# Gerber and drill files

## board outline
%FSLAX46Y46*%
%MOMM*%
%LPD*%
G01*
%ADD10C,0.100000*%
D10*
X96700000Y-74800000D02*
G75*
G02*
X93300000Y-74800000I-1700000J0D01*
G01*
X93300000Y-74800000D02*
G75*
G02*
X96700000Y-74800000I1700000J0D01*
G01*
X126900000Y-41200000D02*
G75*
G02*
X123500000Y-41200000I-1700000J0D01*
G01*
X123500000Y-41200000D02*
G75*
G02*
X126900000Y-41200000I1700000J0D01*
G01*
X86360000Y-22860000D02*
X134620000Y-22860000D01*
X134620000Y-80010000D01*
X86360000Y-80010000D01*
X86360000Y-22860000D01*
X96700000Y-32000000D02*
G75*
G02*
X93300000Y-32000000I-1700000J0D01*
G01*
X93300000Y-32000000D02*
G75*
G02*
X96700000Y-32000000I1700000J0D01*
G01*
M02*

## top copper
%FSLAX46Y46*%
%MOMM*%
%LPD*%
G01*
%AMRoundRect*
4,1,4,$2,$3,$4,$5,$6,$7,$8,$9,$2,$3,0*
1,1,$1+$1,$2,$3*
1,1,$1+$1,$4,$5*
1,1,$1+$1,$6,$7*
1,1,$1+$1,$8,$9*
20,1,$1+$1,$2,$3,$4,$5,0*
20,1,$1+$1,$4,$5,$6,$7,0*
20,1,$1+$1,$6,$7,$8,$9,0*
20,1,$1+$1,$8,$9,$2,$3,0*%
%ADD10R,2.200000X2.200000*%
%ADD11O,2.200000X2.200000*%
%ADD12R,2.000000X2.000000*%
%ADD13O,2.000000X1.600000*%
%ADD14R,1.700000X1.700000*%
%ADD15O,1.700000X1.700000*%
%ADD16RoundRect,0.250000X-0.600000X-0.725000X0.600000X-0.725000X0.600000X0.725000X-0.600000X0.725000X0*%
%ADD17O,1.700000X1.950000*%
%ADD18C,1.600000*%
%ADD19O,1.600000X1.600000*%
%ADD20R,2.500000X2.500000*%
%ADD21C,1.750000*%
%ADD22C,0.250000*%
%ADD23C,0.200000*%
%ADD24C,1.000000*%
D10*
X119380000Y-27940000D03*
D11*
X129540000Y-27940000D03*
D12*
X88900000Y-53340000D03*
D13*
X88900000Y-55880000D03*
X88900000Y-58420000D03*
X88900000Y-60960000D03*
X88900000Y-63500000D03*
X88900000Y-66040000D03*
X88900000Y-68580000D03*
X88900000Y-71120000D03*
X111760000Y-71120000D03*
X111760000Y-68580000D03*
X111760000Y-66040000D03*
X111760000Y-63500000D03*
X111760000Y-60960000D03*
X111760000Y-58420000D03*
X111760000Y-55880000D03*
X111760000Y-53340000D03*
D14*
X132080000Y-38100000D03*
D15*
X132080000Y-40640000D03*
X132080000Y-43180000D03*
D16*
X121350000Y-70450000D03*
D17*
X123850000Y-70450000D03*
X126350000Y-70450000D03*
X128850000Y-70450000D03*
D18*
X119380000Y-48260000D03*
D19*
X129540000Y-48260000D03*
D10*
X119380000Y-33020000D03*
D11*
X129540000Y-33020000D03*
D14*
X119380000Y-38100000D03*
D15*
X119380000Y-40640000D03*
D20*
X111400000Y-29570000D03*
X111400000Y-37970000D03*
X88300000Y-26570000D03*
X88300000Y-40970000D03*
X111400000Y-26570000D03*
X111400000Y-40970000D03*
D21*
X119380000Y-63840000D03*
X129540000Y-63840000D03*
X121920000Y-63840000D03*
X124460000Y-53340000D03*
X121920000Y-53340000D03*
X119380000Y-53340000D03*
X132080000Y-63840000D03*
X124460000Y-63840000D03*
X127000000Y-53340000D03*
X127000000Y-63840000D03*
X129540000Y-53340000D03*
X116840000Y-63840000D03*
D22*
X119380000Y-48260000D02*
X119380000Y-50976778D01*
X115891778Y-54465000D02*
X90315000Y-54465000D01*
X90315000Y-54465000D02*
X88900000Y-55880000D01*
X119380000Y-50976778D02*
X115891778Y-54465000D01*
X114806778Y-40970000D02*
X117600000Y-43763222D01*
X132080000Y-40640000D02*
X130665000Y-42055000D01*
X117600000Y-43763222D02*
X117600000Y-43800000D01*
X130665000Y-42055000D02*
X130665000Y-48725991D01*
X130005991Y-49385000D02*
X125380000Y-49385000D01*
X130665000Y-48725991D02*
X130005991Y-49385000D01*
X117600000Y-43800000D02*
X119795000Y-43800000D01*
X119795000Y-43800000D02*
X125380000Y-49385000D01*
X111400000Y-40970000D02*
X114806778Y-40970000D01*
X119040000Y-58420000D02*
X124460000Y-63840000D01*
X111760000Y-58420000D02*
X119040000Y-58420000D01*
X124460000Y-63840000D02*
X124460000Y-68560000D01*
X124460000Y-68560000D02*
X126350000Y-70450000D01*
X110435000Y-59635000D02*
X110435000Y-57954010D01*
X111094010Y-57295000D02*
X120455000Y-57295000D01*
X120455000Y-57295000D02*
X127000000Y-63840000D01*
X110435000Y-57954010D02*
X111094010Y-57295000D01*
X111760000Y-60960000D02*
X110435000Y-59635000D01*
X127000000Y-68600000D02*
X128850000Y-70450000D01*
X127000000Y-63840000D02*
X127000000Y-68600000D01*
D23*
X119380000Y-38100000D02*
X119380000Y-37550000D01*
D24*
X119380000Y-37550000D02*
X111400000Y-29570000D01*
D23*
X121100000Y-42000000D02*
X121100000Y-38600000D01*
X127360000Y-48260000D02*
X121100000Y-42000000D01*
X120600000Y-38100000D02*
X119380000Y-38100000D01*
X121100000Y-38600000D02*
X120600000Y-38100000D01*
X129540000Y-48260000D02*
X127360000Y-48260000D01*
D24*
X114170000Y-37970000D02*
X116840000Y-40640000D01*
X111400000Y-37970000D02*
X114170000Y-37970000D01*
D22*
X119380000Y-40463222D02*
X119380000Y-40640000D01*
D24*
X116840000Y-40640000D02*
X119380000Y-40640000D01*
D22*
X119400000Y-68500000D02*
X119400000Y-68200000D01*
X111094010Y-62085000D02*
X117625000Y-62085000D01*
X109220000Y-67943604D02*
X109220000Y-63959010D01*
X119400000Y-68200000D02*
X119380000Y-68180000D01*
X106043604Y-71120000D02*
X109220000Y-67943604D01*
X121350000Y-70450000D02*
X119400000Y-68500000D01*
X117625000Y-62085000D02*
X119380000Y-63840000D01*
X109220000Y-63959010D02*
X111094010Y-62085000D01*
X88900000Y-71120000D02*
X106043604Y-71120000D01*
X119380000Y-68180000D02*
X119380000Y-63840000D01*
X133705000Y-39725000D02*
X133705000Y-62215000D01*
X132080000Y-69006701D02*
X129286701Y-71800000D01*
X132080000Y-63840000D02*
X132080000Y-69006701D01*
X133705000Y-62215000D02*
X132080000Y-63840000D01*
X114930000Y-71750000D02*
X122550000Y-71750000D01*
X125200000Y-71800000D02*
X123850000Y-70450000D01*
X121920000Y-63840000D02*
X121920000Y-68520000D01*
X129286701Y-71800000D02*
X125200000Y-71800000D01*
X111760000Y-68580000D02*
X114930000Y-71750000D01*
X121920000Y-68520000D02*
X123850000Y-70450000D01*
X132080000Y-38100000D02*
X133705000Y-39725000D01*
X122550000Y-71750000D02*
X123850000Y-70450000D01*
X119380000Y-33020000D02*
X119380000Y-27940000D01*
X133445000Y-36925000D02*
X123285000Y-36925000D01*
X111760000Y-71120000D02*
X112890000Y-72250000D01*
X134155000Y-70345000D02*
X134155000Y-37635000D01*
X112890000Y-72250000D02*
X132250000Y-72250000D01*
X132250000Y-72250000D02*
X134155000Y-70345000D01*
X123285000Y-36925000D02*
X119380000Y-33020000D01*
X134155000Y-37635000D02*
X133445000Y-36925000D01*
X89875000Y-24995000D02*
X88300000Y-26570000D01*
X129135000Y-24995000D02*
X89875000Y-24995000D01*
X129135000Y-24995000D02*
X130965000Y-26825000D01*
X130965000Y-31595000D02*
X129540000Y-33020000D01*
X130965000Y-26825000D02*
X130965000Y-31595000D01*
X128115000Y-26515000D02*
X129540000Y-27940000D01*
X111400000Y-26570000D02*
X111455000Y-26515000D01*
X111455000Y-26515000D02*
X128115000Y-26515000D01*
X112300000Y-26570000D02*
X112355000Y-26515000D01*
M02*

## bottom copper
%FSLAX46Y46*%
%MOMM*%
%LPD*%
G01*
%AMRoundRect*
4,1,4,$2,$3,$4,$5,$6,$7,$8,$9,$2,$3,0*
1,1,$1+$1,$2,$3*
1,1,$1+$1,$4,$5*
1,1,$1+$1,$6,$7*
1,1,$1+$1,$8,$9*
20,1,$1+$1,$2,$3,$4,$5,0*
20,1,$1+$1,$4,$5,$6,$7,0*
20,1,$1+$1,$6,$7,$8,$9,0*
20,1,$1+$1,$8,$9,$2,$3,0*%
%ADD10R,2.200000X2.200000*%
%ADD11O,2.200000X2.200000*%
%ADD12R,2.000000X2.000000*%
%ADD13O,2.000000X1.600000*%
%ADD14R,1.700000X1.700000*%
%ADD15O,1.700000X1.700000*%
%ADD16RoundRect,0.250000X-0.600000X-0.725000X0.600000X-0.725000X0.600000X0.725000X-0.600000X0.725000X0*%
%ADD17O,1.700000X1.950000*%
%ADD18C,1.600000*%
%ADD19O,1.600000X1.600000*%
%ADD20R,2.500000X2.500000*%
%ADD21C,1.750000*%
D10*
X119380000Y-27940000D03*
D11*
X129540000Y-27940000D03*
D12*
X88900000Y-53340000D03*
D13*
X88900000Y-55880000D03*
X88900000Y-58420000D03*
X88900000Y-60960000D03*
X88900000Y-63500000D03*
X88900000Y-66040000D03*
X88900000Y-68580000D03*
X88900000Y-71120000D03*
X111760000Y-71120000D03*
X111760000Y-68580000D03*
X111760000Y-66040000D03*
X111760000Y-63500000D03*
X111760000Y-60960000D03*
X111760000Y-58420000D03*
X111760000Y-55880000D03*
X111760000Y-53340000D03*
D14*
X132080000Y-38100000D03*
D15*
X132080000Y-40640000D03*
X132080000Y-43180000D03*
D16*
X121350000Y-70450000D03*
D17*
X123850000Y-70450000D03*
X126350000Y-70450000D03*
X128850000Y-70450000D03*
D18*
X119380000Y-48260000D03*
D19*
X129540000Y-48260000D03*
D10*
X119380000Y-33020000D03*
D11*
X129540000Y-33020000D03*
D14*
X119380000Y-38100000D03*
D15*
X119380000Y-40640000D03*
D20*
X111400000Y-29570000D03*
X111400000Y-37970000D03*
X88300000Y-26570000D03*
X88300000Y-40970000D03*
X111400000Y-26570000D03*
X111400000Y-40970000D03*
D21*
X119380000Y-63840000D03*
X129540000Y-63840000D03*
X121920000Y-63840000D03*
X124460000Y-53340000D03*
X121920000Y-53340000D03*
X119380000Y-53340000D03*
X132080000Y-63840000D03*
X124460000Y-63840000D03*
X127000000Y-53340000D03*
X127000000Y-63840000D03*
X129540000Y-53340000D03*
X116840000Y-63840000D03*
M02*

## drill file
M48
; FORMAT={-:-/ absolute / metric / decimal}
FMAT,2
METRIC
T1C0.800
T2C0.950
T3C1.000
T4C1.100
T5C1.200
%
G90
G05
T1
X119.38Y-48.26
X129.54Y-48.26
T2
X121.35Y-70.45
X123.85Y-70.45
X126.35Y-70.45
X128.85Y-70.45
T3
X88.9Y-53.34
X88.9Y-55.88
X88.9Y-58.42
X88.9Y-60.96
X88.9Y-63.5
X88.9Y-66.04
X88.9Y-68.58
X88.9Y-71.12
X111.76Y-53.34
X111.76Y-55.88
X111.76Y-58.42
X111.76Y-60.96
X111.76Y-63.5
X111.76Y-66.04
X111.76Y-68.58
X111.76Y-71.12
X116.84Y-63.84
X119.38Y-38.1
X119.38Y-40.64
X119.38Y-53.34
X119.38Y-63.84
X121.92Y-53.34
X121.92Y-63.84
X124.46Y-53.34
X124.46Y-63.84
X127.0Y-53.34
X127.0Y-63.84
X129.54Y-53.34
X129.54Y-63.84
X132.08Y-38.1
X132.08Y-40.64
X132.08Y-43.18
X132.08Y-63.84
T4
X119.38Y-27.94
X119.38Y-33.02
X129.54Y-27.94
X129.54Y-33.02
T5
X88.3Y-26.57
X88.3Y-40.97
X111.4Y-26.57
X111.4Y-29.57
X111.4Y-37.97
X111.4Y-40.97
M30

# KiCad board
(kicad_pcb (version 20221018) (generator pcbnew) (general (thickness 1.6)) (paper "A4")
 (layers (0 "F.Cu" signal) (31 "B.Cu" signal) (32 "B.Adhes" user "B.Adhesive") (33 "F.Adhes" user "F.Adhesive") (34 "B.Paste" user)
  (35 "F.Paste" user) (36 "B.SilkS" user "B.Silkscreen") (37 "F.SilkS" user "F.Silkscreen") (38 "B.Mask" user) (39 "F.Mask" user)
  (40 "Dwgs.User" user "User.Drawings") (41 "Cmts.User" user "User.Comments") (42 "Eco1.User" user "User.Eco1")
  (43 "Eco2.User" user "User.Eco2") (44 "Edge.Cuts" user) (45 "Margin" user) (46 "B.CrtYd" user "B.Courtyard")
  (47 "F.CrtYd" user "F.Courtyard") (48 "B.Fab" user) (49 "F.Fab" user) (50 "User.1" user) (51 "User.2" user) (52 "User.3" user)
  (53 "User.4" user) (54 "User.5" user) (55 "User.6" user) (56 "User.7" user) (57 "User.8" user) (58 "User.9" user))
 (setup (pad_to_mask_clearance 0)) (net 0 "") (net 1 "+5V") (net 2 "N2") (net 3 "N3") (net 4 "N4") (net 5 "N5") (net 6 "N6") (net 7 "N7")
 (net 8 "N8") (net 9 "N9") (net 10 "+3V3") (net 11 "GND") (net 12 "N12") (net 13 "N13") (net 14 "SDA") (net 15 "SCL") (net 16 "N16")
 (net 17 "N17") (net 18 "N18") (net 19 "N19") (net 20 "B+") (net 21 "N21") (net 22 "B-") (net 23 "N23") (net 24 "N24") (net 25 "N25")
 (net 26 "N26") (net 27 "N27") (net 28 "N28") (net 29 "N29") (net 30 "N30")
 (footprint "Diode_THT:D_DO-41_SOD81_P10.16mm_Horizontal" (layer "F.Cu") (at 119.38 27.94)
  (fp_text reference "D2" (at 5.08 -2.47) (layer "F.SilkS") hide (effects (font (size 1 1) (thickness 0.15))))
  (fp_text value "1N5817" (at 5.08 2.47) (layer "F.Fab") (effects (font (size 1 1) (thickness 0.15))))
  (pad "1" thru_hole rect (at 0 0) (size 2.2 2.2) (drill 1.1) (layers "*.Cu" "*.Mask") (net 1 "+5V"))
  (pad "2" thru_hole oval (at 10.16 0) (size 2.2 2.2) (drill 1.1) (layers "*.Cu" "*.Mask") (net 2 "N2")))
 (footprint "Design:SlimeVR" (layer "F.Cu") (at 124.48 58.59)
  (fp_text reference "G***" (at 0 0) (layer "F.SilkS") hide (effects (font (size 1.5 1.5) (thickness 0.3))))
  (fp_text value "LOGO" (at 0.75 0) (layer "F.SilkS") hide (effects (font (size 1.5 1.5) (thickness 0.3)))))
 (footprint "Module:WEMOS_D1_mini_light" (layer "F.Cu") (at 88.9 53.34)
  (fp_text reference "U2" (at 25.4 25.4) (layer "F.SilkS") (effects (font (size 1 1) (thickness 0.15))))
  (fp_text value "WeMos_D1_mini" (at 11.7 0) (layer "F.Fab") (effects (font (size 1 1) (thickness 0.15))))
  (pad "1" thru_hole rect (at 0 0) (size 2 2) (drill 1) (layers "*.Cu" "*.Mask") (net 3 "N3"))
  (pad "2" thru_hole oval (at 0 2.54) (size 2 1.6) (drill 1) (layers "*.Cu" "*.Mask") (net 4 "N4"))
  (pad "3" thru_hole oval (at 0 5.08) (size 2 1.6) (drill 1) (layers "*.Cu" "*.Mask") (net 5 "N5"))
  (pad "4" thru_hole oval (at 0 7.62) (size 2 1.6) (drill 1) (layers "*.Cu" "*.Mask") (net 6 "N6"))
  (pad "5" thru_hole oval (at 0 10.16) (size 2 1.6) (drill 1) (layers "*.Cu" "*.Mask") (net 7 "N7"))
  (pad "6" thru_hole oval (at 0 12.7) (size 2 1.6) (drill 1) (layers "*.Cu" "*.Mask") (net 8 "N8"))
  (pad "7" thru_hole oval (at 0 15.24) (size 2 1.6) (drill 1) (layers "*.Cu" "*.Mask") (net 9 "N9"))
  (pad "8" thru_hole oval (at 0 17.78) (size 2 1.6) (drill 1) (layers "*.Cu" "*.Mask") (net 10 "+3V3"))
  (pad "9" thru_hole oval (at 22.86 17.78) (size 2 1.6) (drill 1) (layers "*.Cu" "*.Mask") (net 1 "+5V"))
  (pad "10" thru_hole oval (at 22.86 15.24) (size 2 1.6) (drill 1) (layers "*.Cu" "*.Mask") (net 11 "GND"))
  (pad "11" thru_hole oval (at 22.86 12.7) (size 2 1.6) (drill 1) (layers "*.Cu" "*.Mask") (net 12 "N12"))
  (pad "12" thru_hole oval (at 22.86 10.16) (size 2 1.6) (drill 1) (layers "*.Cu" "*.Mask") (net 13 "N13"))
  (pad "13" thru_hole oval (at 22.86 7.62) (size 2 1.6) (drill 1) (layers "*.Cu" "*.Mask") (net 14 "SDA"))
  (pad "14" thru_hole oval (at 22.86 5.08) (size 2 1.6) (drill 1) (layers "*.Cu" "*.Mask") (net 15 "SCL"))
  (pad "15" thru_hole oval (at 22.86 2.54) (size 2 1.6) (drill 1) (layers "*.Cu" "*.Mask") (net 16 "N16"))
  (pad "16" thru_hole oval (at 22.86 0) (size 2 1.6) (drill 1) (layers "*.Cu" "*.Mask") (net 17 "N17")))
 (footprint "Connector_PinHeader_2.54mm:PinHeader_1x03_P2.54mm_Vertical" (layer "F.Cu") (at 132.08 38.1)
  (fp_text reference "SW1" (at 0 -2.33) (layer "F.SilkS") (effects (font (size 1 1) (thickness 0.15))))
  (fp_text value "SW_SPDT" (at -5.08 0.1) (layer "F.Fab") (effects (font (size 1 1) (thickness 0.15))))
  (pad "1" thru_hole rect (at 0 0) (size 1.7 1.7) (drill 1) (layers "*.Cu" "*.Mask") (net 11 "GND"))
  (pad "2" thru_hole oval (at 0 2.54) (size 1.7 1.7) (drill 1) (layers "*.Cu" "*.Mask") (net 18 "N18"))
  (pad "3" thru_hole oval (at 0 5.08) (size 1.7 1.7) (drill 1) (layers "*.Cu" "*.Mask") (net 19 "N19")))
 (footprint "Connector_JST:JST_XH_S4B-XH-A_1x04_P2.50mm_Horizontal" (layer "F.Cu") (at 121.35 70.45)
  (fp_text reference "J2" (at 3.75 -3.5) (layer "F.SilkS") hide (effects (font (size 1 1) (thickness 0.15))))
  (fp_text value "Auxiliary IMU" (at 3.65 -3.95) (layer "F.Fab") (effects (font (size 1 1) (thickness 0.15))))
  (pad "1" thru_hole roundrect (at 0 0) (size 1.7 1.95) (drill 0.95) (layers "*.Cu" "*.Mask") (roundrect_rratio 0.1470588235)
   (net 10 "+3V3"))
  (pad "2" thru_hole oval (at 2.5 0) (size 1.7 1.95) (drill 0.95) (layers "*.Cu" "*.Mask") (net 11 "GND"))
  (pad "3" thru_hole oval (at 5 0) (size 1.7 1.95) (drill 0.95) (layers "*.Cu" "*.Mask") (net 15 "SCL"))
  (pad "4" thru_hole oval (at 7.5 0) (size 1.7 1.95) (drill 0.95) (layers "*.Cu" "*.Mask") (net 14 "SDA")))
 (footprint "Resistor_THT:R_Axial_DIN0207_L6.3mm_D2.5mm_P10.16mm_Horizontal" (layer "F.Cu") (at 119.38 48.26)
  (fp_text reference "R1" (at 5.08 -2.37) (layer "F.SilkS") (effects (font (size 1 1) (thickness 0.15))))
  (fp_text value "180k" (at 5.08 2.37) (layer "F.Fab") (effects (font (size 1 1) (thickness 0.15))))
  (pad "1" thru_hole circle (at 0 0) (size 1.6 1.6) (drill 0.8) (layers "*.Cu" "*.Mask") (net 4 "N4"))
  (pad "2" thru_hole oval (at 10.16 0) (size 1.6 1.6) (drill 0.8) (layers "*.Cu" "*.Mask") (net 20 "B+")))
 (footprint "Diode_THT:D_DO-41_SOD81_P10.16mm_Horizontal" (layer "F.Cu") (at 119.38 33.02)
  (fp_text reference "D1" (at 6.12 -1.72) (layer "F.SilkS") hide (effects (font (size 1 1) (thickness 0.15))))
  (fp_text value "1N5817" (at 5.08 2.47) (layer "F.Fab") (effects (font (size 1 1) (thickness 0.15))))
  (pad "1" thru_hole rect (at 0 0) (size 2.2 2.2) (drill 1.1) (layers "*.Cu" "*.Mask") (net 1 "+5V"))
  (pad "2" thru_hole oval (at 10.16 0) (size 2.2 2.2) (drill 1.1) (layers "*.Cu" "*.Mask") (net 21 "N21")))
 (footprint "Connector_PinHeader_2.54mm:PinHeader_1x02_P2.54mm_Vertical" (layer "F.Cu") (at 119.38 38.1)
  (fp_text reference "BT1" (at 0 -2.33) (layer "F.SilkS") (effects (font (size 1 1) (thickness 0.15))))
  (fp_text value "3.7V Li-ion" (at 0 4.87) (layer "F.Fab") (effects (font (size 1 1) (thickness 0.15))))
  (pad "1" thru_hole rect (at 0 0) (size 1.7 1.7) (drill 1) (layers "*.Cu" "*.Mask") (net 20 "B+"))
  (pad "2" thru_hole oval (at 0 2.54) (size 1.7 1.7) (drill 1) (layers "*.Cu" "*.Mask") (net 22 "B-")))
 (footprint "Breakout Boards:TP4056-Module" (layer "F.Cu") (at 100.7 33.02)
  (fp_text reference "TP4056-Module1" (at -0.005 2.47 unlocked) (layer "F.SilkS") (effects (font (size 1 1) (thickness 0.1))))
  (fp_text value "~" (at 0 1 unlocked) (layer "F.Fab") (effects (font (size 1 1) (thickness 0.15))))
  (pad "B+" thru_hole rect (at 10.7 -3.45) (size 2.5 2.5) (drill 1.2) (layers "*.Cu" "*.Mask" "Eco1.User") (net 20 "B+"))
  (pad "B-" thru_hole rect (at 10.7 4.95) (size 2.5 2.5) (drill 1.2) (layers "*.Cu" "*.Mask" "Eco1.User") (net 22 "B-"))
  (pad "IN+" thru_hole rect (at -12.4 -6.45) (size 2.5 2.5) (drill 1.2) (layers "*.Cu" "*.Mask" "Eco1.User") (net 21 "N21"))
  (pad "IN-" thru_hole rect (at -12.4 7.95) (size 2.5 2.5) (drill 1.2) (layers "*.Cu" "*.Mask" "Eco1.User") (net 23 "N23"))
  (pad "OUT+" thru_hole rect (at 10.7 -6.45) (size 2.5 2.5) (drill 1.2) (layers "*.Cu" "*.Mask" "Eco1.User") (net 2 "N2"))
  (pad "OUT-" thru_hole rect (at 10.7 7.95) (size 2.5 2.5) (drill 1.2) (layers "*.Cu" "*.Mask" "Eco1.User") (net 18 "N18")))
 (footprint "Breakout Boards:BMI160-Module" (layer "F.Cu") (at 124.47 57.245)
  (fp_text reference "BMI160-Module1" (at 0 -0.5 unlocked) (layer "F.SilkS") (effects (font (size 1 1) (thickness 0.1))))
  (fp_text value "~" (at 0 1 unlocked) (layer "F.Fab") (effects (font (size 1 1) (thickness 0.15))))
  (pad "3V3" thru_hole circle (at -5.09 6.595) (size 1.75 1.75) (drill 1) (layers "*.Cu" "*.Mask" "Eco1.User") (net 10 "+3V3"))
  (pad "CS" thru_hole circle (at 5.07 6.595) (size 1.75 1.75) (drill 1) (layers "*.Cu" "*.Mask" "Eco1.User") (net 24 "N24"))
  (pad "GND" thru_hole circle (at -2.55 6.595) (size 1.75 1.75) (drill 1) (layers "*.Cu" "*.Mask" "Eco1.User") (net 11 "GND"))
  (pad "INT1" thru_hole circle (at -0.01 -3.905) (size 1.75 1.75) (drill 1) (layers "*.Cu" "*.Mask" "Eco1.User") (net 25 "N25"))
  (pad "INT2" thru_hole circle (at -2.55 -3.905) (size 1.75 1.75) (drill 1) (layers "*.Cu" "*.Mask" "Eco1.User") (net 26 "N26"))
  (pad "OCS" thru_hole circle (at -5.09 -3.905) (size 1.75 1.75) (drill 1) (layers "*.Cu" "*.Mask" "Eco1.User") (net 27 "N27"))
  (pad "SAO" thru_hole circle (at 7.61 6.595) (size 1.75 1.75) (drill 1) (layers "*.Cu" "*.Mask" "Eco1.User") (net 11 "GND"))
  (pad "SCL" thru_hole circle (at -0.01 6.595) (size 1.75 1.75) (drill 1) (layers "*.Cu" "*.Mask" "Eco1.User") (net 15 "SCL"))
  (pad "SCX" thru_hole circle (at 2.53 -3.905) (size 1.75 1.75) (drill 1) (layers "*.Cu" "*.Mask" "Eco1.User") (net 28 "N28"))
  (pad "SDA" thru_hole circle (at 2.53 6.595) (size 1.75 1.75) (drill 1) (layers "*.Cu" "*.Mask" "Eco1.User") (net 14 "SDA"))
  (pad "SDX" thru_hole circle (at 5.07 -3.905) (size 1.75 1.75) (drill 1) (layers "*.Cu" "*.Mask" "Eco1.User") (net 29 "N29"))
  (pad "VIN" thru_hole circle (at -7.63 6.595) (size 1.75 1.75) (drill 1) (layers "*.Cu" "*.Mask" "Eco1.User") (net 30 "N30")))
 (gr_circle (center 95 74.8) (end 93.3 74.8) (stroke (width 0.1) (type default)) (fill none) (layer "Edge.Cuts"))
 (gr_circle (center 125.2 41.2) (end 126.9 41.2) (stroke (width 0.1) (type default)) (fill none) (layer "Edge.Cuts"))
 (gr_rect (start 86.36 22.86) (end 134.62 80.01) (stroke (width 0.1) (type default)) (fill none) (layer "Edge.Cuts"))
 (gr_circle (center 95 32) (end 93.3 32) (stroke (width 0.1) (type default)) (fill none) (layer "Edge.Cuts"))
 (segment (start 119.38 48.26) (end 119.38 50.976778) (width 0.25) (layer "F.Cu") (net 4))
 (segment (start 115.891778 54.465) (end 90.315 54.465) (width 0.25) (layer "F.Cu") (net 4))
 (segment (start 90.315 54.465) (end 88.9 55.88) (width 0.25) (layer "F.Cu") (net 4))
 (segment (start 119.38 50.976778) (end 115.891778 54.465) (width 0.25) (layer "F.Cu") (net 4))
 (segment (start 114.806778 40.97) (end 117.6 43.763222) (width 0.25) (layer "F.Cu") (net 18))
 (segment (start 132.08 40.64) (end 130.665 42.055) (width 0.25) (layer "F.Cu") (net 18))
 (segment (start 117.6 43.763222) (end 117.6 43.8) (width 0.25) (layer "F.Cu") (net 18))
 (segment (start 130.665 42.055) (end 130.665 48.725991) (width 0.25) (layer "F.Cu") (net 18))
 (segment (start 130.005991 49.385) (end 125.38 49.385) (width 0.25) (layer "F.Cu") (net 18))
 (segment (start 130.665 48.725991) (end 130.005991 49.385) (width 0.25) (layer "F.Cu") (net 18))
 (segment (start 117.6 43.8) (end 119.795 43.8) (width 0.25) (layer "F.Cu") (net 18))
 (segment (start 119.795 43.8) (end 125.38 49.385) (width 0.25) (layer "F.Cu") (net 18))
 (segment (start 111.4 40.97) (end 114.806778 40.97) (width 0.25) (layer "F.Cu") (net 18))
 (segment (start 119.04 58.42) (end 124.46 63.84) (width 0.25) (layer "F.Cu") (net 15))
 (segment (start 111.76 58.42) (end 119.04 58.42) (width 0.25) (layer "F.Cu") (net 15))
 (segment (start 124.46 63.84) (end 124.46 68.56) (width 0.25) (layer "F.Cu") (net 15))
 (segment (start 124.46 68.56) (end 126.35 70.45) (width 0.25) (layer "F.Cu") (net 15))
 (segment (start 110.435 59.635) (end 110.435 57.95401) (width 0.25) (layer "F.Cu") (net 14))
 (segment (start 111.09401 57.295) (end 120.455 57.295) (width 0.25) (layer "F.Cu") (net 14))
 (segment (start 120.455 57.295) (end 127 63.84) (width 0.25) (layer "F.Cu") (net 14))
 (segment (start 110.435 57.95401) (end 111.09401 57.295) (width 0.25) (layer "F.Cu") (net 14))
 (segment (start 111.76 60.96) (end 110.435 59.635) (width 0.25) (layer "F.Cu") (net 14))
 (segment (start 127 68.6) (end 128.85 70.45) (width 0.25) (layer "F.Cu") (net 14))
 (segment (start 127 63.84) (end 127 68.6) (width 0.25) (layer "F.Cu") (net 14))
 (segment (start 119.38 38.1) (end 119.38 37.55) (width 0.2) (layer "F.Cu") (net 20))
 (segment (start 119.38 37.55) (end 111.4 29.57) (width 1) (layer "F.Cu") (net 20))
 (segment (start 121.1 42) (end 121.1 38.6) (width 0.2) (layer "F.Cu") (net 20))
 (segment (start 127.36 48.26) (end 121.1 42) (width 0.2) (layer "F.Cu") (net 20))
 (segment (start 120.6 38.1) (end 119.38 38.1) (width 0.2) (layer "F.Cu") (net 20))
 (segment (start 121.1 38.6) (end 120.6 38.1) (width 0.2) (layer "F.Cu") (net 20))
 (segment (start 129.54 48.26) (end 127.36 48.26) (width 0.2) (layer "F.Cu") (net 20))
 (segment (start 114.17 37.97) (end 116.84 40.64) (width 1) (layer "F.Cu") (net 22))
 (segment (start 111.4 37.97) (end 114.17 37.97) (width 1) (layer "F.Cu") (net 22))
 (segment (start 119.38 40.463222) (end 119.38 40.64) (width 0.25) (layer "F.Cu") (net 22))
 (segment (start 116.84 40.64) (end 119.38 40.64) (width 1) (layer "F.Cu") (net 22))
 (segment (start 119.4 68.5) (end 119.4 68.2) (width 0.25) (layer "F.Cu") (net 10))
 (segment (start 111.09401 62.085) (end 117.625 62.085) (width 0.25) (layer "F.Cu") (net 10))
 (segment (start 109.22 67.943604) (end 109.22 63.95901) (width 0.25) (layer "F.Cu") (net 10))
 (segment (start 119.4 68.2) (end 119.38 68.18) (width 0.25) (layer "F.Cu") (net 10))
 (segment (start 106.043604 71.12) (end 109.22 67.943604) (width 0.25) (layer "F.Cu") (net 10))
 (segment (start 121.35 70.45) (end 119.4 68.5) (width 0.25) (layer "F.Cu") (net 10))
 (segment (start 117.625 62.085) (end 119.38 63.84) (width 0.25) (layer "F.Cu") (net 10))
 (segment (start 109.22 63.95901) (end 111.09401 62.085) (width 0.25) (layer "F.Cu") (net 10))
 (segment (start 88.9 71.12) (end 106.043604 71.12) (width 0.25) (layer "F.Cu") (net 10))
 (segment (start 119.38 68.18) (end 119.38 63.84) (width 0.25) (layer "F.Cu") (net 10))
 (segment (start 133.705 39.725) (end 133.705 62.215) (width 0.25) (layer "F.Cu") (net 11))
 (segment (start 132.08 69.006701) (end 129.286701 71.8) (width 0.25) (layer "F.Cu") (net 11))
 (segment (start 132.08 63.84) (end 132.08 69.006701) (width 0.25) (layer "F.Cu") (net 11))
 (segment (start 133.705 62.215) (end 132.08 63.84) (width 0.25) (layer "F.Cu") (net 11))
 (segment (start 114.93 71.75) (end 122.55 71.75) (width 0.25) (layer "F.Cu") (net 11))
 (segment (start 125.2 71.8) (end 123.85 70.45) (width 0.25) (layer "F.Cu") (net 11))
 (segment (start 121.92 63.84) (end 121.92 68.52) (width 0.25) (layer "F.Cu") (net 11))
 (segment (start 129.286701 71.8) (end 125.2 71.8) (width 0.25) (layer "F.Cu") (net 11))
 (segment (start 111.76 68.58) (end 114.93 71.75) (width 0.25) (layer "F.Cu") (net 11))
 (segment (start 121.92 68.52) (end 123.85 70.45) (width 0.25) (layer "F.Cu") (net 11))
 (segment (start 132.08 38.1) (end 133.705 39.725) (width 0.25) (layer "F.Cu") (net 11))
 (segment (start 122.55 71.75) (end 123.85 70.45) (width 0.25) (layer "F.Cu") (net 11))
 (segment (start 119.38 33.02) (end 119.38 27.94) (width 0.25) (layer "F.Cu") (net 1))
 (segment (start 133.445 36.925) (end 123.285 36.925) (width 0.25) (layer "F.Cu") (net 1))
 (segment (start 111.76 71.12) (end 112.89 72.25) (width 0.25) (layer "F.Cu") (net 1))
 (segment (start 134.155 70.345) (end 134.155 37.635) (width 0.25) (layer "F.Cu") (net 1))
 (segment (start 112.89 72.25) (end 132.25 72.25) (width 0.25) (layer "F.Cu") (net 1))
 (segment (start 132.25 72.25) (end 134.155 70.345) (width 0.25) (layer "F.Cu") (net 1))
 (segment (start 123.285 36.925) (end 119.38 33.02) (width 0.25) (layer "F.Cu") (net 1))
 (segment (start 134.155 37.635) (end 133.445 36.925) (width 0.25) (layer "F.Cu") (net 1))
 (segment (start 89.875 24.995) (end 88.3 26.57) (width 0.25) (layer "F.Cu") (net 21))
 (segment (start 129.135 24.995) (end 89.875 24.995) (width 0.25) (layer "F.Cu") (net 21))
 (segment (start 129.135 24.995) (end 130.965 26.825) (width 0.25) (layer "F.Cu") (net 21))
 (segment (start 130.965 31.595) (end 129.54 33.02) (width 0.25) (layer "F.Cu") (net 21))
 (segment (start 130.965 26.825) (end 130.965 31.595) (width 0.25) (layer "F.Cu") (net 21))
 (segment (start 128.115 26.515) (end 129.54 27.94) (width 0.25) (layer "F.Cu") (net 2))
 (segment (start 111.4 26.57) (end 111.455 26.515) (width 0.25) (layer "F.Cu") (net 2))
 (segment (start 111.455 26.515) (end 128.115 26.515) (width 0.25) (layer "F.Cu") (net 2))
 (segment (start 112.3 26.57) (end 112.355 26.515) (width 0.25) (layer "F.Cu") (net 2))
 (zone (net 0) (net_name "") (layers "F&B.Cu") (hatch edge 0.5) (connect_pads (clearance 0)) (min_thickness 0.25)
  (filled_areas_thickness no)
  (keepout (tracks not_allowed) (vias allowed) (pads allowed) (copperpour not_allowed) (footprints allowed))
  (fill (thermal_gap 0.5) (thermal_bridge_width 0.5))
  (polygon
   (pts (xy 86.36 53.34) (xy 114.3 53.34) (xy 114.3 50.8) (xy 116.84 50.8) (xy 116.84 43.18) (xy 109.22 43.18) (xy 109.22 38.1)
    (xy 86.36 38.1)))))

